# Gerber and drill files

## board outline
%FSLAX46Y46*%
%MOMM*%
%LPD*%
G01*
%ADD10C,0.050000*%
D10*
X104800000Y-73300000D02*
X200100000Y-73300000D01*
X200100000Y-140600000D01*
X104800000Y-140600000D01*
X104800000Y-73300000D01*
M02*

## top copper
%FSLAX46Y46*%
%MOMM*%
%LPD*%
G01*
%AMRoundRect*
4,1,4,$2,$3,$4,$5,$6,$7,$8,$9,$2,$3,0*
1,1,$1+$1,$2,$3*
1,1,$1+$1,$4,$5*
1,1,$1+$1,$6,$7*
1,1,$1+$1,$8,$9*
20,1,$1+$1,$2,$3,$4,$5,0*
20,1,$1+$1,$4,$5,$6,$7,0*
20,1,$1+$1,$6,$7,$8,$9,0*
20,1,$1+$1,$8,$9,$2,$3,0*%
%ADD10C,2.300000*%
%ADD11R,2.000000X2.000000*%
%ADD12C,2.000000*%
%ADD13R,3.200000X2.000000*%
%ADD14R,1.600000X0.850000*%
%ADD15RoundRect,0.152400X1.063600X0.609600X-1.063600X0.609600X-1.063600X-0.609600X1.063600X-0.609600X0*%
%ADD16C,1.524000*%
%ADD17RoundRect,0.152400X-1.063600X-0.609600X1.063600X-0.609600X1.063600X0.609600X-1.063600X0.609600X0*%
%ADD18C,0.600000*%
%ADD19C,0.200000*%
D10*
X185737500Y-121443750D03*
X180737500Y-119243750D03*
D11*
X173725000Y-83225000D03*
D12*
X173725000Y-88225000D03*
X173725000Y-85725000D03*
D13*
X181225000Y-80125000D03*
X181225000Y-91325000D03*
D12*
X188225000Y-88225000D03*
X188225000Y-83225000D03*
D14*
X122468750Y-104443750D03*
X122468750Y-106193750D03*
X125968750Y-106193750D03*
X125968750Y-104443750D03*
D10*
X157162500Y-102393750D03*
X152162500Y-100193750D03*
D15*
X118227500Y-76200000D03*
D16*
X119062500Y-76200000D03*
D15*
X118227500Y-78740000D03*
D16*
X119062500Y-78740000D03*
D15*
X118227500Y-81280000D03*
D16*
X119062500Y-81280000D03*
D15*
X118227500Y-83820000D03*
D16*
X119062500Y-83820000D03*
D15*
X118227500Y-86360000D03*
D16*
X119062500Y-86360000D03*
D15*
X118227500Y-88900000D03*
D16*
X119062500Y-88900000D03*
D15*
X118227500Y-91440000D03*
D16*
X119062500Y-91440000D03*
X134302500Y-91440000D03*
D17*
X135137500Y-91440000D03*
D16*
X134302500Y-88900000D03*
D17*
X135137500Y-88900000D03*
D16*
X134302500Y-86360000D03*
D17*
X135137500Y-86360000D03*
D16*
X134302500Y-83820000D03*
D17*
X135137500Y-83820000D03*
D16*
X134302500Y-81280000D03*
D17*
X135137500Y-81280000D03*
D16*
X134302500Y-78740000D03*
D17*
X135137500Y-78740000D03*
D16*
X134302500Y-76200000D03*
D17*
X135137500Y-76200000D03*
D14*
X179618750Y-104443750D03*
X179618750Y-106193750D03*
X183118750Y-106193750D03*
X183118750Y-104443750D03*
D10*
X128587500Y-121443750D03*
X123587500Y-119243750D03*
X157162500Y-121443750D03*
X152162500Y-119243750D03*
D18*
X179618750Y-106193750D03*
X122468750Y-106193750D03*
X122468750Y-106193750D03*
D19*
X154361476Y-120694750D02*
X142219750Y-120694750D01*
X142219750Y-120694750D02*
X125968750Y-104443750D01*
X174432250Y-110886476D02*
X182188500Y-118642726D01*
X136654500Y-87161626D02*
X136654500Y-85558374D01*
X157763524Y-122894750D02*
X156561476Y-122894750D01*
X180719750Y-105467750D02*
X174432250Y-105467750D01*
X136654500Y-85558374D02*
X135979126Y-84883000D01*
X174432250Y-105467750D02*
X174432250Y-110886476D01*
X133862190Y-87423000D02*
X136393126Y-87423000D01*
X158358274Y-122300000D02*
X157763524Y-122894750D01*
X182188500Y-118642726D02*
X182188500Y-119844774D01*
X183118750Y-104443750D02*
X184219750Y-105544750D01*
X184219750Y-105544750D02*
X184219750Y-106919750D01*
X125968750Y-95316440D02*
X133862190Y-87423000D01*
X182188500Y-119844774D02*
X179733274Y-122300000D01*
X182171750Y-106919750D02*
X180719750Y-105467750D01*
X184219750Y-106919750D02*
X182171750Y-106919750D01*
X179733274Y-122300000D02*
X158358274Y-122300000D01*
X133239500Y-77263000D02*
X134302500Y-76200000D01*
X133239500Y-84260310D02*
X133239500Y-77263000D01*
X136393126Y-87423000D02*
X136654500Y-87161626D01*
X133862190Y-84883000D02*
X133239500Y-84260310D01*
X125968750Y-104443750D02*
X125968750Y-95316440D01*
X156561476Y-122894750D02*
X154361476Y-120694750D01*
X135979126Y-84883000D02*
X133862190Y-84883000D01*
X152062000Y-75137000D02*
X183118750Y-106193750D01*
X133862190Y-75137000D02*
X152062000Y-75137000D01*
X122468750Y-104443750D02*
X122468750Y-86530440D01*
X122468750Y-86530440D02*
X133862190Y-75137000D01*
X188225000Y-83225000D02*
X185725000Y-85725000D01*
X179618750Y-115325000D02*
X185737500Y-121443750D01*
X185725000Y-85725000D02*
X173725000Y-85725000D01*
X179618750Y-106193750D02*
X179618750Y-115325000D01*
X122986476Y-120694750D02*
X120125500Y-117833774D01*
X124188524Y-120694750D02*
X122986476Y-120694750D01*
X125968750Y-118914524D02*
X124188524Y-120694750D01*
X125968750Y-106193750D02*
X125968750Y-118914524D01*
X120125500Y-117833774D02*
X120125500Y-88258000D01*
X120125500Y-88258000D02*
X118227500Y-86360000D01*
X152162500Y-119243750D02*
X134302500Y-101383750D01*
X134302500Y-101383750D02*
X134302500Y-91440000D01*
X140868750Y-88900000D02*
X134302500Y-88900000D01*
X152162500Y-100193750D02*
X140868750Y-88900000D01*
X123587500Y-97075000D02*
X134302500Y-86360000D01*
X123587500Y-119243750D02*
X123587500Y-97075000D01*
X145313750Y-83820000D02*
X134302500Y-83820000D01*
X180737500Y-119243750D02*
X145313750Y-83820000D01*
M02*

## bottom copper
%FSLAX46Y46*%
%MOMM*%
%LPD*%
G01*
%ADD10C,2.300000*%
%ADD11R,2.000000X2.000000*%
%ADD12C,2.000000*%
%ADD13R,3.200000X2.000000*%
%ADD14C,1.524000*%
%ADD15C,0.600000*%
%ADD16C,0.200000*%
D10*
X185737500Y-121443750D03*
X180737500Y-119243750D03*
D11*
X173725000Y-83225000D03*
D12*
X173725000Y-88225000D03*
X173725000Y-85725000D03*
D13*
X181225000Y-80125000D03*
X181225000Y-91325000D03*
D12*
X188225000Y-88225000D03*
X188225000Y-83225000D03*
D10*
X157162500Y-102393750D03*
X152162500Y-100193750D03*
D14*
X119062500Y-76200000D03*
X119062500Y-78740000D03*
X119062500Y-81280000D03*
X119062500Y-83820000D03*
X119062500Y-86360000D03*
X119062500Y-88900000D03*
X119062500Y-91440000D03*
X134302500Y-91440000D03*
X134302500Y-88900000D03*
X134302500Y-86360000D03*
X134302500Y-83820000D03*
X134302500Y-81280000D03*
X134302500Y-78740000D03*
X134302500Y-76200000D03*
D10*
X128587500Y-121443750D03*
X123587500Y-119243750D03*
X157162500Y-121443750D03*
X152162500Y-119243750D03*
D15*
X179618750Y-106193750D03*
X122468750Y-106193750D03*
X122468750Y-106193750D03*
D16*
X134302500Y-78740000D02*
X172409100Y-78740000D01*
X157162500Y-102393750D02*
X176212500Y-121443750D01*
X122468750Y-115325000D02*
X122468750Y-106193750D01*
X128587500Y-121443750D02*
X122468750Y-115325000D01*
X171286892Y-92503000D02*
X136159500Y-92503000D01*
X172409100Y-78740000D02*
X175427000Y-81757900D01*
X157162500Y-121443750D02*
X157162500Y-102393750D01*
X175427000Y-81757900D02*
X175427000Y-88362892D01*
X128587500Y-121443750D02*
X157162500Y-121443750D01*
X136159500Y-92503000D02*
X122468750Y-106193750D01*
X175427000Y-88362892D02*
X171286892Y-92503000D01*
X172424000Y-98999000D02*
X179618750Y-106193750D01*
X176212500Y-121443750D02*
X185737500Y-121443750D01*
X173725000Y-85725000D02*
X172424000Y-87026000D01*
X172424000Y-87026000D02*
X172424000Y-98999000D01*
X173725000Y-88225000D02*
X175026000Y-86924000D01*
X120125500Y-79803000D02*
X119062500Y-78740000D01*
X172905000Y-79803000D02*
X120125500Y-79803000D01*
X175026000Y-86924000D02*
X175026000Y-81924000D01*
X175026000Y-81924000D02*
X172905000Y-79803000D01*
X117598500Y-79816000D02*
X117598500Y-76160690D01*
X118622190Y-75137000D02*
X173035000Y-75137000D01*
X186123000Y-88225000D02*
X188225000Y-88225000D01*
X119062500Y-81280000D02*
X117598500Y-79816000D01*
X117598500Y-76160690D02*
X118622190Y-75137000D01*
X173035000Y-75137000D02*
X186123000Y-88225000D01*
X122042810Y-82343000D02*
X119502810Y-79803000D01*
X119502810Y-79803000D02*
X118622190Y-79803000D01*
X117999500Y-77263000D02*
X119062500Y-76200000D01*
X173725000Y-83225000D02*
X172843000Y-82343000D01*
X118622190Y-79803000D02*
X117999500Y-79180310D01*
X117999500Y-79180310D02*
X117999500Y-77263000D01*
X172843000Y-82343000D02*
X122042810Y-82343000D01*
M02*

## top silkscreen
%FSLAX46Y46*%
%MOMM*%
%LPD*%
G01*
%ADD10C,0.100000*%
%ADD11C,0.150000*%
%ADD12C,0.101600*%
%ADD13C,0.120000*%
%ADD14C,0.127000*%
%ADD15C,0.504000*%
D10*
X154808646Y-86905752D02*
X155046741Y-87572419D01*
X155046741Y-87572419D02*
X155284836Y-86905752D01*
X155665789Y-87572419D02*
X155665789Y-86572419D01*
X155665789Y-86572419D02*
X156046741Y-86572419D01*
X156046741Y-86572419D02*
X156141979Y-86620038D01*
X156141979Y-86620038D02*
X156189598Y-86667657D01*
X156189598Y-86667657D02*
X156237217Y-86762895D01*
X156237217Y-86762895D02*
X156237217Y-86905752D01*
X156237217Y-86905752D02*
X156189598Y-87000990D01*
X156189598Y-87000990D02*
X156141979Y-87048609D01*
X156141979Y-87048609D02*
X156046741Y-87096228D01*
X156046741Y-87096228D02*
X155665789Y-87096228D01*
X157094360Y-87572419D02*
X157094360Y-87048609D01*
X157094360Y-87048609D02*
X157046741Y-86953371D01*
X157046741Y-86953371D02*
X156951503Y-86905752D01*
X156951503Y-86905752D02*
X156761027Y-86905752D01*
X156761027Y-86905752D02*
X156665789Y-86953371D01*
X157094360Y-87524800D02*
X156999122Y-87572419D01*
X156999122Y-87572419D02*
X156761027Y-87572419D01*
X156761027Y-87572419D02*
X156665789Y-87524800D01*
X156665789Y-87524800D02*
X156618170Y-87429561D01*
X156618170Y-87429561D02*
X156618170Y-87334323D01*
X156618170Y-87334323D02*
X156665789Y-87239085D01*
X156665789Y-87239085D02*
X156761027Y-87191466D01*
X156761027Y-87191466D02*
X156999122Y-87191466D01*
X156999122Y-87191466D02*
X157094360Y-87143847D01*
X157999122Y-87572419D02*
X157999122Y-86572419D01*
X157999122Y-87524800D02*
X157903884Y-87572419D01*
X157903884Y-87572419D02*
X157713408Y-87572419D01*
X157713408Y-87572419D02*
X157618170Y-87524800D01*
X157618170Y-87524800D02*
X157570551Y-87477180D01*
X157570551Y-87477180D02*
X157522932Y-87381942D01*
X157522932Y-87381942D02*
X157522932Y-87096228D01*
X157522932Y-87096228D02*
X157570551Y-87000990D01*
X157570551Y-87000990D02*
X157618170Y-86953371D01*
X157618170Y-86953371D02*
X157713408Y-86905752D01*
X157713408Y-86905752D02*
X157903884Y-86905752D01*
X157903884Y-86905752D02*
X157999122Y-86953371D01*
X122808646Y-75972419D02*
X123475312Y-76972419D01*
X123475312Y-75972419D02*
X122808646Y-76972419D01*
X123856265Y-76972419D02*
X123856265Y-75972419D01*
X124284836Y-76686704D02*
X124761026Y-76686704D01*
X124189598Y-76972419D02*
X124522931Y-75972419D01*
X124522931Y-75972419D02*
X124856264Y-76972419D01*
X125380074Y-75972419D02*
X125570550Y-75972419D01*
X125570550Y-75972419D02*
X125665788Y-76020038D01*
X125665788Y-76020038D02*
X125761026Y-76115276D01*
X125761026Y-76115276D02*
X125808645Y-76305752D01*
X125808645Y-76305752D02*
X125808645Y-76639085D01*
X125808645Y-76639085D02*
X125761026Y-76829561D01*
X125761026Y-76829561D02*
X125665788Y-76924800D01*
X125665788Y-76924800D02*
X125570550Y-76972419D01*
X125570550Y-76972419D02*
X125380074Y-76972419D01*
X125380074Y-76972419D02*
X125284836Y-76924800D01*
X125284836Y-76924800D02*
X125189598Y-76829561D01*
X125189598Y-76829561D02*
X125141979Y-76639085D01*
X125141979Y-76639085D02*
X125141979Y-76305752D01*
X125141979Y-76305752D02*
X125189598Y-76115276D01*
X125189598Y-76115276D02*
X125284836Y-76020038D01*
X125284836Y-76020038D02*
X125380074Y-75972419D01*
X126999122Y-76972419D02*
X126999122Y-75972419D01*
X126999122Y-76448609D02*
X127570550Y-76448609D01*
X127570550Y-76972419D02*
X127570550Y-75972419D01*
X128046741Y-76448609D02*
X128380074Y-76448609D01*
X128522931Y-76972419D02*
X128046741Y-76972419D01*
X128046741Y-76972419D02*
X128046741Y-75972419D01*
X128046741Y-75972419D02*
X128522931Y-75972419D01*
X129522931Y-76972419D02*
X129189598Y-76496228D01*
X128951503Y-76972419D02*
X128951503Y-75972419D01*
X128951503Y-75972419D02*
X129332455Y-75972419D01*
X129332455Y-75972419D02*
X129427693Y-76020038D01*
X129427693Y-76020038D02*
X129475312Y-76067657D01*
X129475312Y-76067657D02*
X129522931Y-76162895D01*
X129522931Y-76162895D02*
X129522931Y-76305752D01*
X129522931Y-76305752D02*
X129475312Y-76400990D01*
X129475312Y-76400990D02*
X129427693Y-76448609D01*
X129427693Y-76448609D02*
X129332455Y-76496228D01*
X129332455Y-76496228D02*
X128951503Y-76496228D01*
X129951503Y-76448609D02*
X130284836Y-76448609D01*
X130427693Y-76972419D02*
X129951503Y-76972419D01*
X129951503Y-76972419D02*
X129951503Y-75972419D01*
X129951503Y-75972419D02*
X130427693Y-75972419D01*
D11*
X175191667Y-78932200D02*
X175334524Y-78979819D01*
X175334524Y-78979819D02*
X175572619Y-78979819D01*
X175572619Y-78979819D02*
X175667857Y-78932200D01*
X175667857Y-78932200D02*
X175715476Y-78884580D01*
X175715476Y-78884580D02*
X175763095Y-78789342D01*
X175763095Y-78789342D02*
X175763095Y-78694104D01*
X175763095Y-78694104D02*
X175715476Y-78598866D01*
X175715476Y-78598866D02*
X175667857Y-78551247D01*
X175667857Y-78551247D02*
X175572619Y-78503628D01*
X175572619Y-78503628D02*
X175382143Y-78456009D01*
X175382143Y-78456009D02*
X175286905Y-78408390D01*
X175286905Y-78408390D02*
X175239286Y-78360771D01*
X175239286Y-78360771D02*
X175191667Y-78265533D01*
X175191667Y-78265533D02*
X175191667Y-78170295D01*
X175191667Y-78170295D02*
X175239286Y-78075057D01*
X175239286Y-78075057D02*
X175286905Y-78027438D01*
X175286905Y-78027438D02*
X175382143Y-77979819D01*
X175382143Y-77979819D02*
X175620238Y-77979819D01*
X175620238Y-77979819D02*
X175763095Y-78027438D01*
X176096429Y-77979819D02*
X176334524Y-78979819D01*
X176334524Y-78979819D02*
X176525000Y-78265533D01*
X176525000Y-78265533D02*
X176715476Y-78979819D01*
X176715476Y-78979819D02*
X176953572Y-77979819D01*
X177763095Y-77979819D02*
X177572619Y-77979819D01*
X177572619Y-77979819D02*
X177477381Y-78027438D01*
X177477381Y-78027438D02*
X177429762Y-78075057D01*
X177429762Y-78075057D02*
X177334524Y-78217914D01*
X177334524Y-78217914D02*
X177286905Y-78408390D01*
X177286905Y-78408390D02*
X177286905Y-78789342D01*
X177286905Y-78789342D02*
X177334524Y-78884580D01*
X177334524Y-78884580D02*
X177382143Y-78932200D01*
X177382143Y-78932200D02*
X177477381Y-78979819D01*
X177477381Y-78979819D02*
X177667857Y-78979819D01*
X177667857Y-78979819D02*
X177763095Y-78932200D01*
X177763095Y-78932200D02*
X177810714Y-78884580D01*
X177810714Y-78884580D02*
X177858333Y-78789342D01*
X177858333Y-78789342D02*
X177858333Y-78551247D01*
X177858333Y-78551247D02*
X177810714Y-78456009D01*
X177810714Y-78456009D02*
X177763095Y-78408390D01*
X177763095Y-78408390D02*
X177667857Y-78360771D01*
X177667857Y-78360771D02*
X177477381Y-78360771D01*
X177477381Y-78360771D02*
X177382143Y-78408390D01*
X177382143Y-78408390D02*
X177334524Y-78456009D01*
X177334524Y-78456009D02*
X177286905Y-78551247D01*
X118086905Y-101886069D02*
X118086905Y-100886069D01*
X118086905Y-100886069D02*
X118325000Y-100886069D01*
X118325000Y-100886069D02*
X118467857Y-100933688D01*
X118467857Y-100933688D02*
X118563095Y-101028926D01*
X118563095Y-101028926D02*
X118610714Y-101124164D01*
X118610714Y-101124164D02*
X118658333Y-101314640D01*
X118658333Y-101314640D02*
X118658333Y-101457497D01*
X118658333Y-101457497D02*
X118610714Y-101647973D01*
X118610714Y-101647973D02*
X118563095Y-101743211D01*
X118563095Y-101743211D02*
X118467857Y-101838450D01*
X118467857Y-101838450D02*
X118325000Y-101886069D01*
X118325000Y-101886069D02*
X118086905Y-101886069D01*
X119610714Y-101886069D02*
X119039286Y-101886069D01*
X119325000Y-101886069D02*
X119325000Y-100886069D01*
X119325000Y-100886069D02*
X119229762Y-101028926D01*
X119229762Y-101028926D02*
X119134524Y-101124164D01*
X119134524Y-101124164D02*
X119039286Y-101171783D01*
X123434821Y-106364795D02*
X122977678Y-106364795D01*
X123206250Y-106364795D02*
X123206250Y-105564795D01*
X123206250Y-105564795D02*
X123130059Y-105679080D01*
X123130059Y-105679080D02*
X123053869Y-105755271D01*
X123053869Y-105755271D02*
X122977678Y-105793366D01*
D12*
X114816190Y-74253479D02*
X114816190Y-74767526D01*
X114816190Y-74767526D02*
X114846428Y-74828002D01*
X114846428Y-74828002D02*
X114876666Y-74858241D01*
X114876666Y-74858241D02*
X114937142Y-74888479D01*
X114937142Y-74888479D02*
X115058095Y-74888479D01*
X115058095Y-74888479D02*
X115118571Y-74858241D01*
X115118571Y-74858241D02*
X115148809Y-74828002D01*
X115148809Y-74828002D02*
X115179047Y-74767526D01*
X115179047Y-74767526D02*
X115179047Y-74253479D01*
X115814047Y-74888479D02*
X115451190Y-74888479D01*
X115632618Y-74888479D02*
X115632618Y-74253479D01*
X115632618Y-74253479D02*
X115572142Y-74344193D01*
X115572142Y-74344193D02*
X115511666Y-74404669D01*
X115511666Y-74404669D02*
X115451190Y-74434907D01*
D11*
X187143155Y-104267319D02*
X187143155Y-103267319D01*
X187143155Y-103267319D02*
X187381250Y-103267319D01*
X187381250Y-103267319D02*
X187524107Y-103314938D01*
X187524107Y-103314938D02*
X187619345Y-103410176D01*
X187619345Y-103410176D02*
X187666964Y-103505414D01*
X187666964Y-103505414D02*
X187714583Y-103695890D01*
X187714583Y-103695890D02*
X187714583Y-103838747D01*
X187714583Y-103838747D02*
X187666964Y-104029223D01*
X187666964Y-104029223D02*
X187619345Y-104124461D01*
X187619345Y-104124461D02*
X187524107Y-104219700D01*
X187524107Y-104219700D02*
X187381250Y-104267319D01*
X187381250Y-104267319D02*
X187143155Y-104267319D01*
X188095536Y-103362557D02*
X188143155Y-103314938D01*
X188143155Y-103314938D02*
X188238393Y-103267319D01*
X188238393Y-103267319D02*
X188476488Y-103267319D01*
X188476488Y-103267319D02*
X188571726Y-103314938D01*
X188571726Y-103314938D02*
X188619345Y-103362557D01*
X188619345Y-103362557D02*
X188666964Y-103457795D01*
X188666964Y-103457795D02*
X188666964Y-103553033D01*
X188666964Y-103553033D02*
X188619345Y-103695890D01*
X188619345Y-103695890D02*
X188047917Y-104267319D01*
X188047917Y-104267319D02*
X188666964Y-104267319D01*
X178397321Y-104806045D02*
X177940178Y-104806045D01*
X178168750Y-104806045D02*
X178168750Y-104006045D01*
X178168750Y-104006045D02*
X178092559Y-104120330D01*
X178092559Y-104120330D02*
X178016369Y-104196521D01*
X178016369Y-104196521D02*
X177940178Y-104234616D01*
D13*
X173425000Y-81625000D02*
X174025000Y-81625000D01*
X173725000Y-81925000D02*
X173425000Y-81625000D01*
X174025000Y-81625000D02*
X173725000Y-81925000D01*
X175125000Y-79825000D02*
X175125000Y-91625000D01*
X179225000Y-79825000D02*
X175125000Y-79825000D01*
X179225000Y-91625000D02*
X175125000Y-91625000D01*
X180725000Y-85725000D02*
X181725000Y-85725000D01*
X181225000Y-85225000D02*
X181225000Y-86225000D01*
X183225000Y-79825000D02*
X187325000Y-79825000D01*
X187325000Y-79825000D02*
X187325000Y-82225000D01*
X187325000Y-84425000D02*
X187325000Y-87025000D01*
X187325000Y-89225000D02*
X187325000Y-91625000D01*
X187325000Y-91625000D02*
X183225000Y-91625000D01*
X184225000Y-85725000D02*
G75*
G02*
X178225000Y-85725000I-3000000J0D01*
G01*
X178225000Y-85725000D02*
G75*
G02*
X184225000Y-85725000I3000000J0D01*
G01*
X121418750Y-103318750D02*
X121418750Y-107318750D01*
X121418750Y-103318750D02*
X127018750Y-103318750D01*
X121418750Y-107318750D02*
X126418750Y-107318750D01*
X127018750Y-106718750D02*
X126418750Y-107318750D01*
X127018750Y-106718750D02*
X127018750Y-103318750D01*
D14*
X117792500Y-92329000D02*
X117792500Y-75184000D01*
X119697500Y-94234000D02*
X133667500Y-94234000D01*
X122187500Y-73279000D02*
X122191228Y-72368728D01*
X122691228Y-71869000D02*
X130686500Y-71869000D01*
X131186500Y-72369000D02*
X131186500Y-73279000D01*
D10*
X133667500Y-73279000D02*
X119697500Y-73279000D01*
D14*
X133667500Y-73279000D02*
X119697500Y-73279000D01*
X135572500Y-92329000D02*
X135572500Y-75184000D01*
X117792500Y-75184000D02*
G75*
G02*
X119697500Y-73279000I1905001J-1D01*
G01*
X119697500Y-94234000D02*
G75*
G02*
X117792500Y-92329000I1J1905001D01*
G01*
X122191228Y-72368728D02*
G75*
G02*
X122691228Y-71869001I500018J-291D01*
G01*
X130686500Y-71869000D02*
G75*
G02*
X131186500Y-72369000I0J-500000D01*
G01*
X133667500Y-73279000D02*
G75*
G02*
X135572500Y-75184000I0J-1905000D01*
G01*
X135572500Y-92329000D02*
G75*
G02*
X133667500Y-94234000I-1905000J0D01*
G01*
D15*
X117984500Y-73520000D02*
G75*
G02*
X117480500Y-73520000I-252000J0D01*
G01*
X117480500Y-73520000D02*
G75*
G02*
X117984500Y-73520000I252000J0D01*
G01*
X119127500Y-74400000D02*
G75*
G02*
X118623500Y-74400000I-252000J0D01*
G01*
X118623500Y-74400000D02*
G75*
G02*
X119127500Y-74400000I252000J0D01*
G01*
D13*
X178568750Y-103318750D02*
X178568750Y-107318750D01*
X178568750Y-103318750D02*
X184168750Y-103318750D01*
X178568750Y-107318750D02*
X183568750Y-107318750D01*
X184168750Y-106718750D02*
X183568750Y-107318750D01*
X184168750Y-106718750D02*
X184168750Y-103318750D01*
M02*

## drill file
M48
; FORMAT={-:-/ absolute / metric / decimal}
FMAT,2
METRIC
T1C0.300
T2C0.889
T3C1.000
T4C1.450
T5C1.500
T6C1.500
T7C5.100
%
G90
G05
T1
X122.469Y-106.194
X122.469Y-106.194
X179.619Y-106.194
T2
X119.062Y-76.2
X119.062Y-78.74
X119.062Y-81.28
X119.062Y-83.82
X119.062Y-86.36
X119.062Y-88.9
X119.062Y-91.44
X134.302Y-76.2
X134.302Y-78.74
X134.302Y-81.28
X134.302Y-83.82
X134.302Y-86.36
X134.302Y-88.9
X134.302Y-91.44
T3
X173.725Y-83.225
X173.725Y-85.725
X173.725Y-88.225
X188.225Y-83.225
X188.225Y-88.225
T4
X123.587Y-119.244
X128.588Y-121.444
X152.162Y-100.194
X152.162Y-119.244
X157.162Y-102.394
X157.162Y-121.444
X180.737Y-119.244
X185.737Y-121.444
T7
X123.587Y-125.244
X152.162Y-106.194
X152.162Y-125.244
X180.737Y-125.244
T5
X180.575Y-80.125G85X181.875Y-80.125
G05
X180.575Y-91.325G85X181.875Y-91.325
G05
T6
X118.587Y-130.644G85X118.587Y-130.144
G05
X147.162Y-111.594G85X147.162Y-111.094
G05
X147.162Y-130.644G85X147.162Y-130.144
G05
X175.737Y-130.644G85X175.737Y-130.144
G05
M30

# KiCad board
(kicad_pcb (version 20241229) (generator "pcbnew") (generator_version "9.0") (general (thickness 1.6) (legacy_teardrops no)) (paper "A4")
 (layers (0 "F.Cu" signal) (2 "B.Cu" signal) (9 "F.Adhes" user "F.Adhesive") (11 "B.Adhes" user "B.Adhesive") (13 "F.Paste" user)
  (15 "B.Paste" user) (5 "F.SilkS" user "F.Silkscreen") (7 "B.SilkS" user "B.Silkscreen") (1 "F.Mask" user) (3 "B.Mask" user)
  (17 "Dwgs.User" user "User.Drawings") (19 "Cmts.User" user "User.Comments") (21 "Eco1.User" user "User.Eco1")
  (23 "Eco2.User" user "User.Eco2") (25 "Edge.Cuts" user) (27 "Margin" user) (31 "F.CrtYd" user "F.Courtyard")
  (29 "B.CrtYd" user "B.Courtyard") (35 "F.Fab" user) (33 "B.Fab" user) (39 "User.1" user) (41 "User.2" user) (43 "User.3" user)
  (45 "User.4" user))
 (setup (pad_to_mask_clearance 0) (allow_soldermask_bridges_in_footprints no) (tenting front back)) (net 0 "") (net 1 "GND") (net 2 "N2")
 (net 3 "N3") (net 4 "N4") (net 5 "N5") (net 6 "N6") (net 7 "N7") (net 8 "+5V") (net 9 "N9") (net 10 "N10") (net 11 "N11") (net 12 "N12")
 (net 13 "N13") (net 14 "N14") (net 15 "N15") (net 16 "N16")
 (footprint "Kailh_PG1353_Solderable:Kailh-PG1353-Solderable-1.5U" (layer "F.Cu") (at 180.7375 125.24375)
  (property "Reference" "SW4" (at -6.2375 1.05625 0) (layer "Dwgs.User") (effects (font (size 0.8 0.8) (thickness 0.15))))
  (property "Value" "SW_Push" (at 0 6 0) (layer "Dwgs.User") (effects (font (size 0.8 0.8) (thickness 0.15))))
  (pad "" np_thru_hole oval (at -5 5.15 180) (size 1.5 2) (drill oval 1.5 2) (layers "*.Cu" "*.Mask"))
  (pad "" np_thru_hole circle (at 0 0 180) (size 5 5) (drill 5.1) (layers "*.Cu" "*.Mask"))
  (pad "1" thru_hole circle (at 5 -3.8 180) (size 2.3 2.3) (drill 1.45) (layers "*.Cu" "B.Mask") (remove_unused_layers no) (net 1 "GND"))
  (pad "2" thru_hole circle (at 0 -6 180) (size 2.3 2.3) (drill 1.45) (layers "*.Cu" "B.Mask") (remove_unused_layers no) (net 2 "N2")))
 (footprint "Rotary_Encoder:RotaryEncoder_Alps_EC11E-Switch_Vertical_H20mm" (layer "F.Cu") (at 173.725 83.225)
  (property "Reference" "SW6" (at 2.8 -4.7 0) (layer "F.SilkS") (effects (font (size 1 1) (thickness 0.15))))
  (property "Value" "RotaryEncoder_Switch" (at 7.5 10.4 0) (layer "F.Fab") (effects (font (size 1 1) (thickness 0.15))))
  (fp_line (start -0.3 -1.6) (end 0.3 -1.6) (stroke (width 0.12) (type solid)) (layer "F.SilkS"))
  (fp_line (start 0 -1.3) (end -0.3 -1.6) (stroke (width 0.12) (type solid)) (layer "F.SilkS"))
  (fp_line (start 0.3 -1.6) (end 0 -1.3) (stroke (width 0.12) (type solid)) (layer "F.SilkS"))
  (fp_line (start 1.4 -3.4) (end 1.4 8.4) (stroke (width 0.12) (type solid)) (layer "F.SilkS"))
  (fp_line (start 5.5 -3.4) (end 1.4 -3.4) (stroke (width 0.12) (type solid)) (layer "F.SilkS"))
  (fp_line (start 5.5 8.4) (end 1.4 8.4) (stroke (width 0.12) (type solid)) (layer "F.SilkS"))
  (fp_line (start 7 2.5) (end 8 2.5) (stroke (width 0.12) (type solid)) (layer "F.SilkS"))
  (fp_line (start 7.5 2) (end 7.5 3) (stroke (width 0.12) (type solid)) (layer "F.SilkS"))
  (fp_line (start 9.5 -3.4) (end 13.6 -3.4) (stroke (width 0.12) (type solid)) (layer "F.SilkS"))
  (fp_line (start 13.6 -3.4) (end 13.6 -1) (stroke (width 0.12) (type solid)) (layer "F.SilkS"))
  (fp_line (start 13.6 1.2) (end 13.6 3.8) (stroke (width 0.12) (type solid)) (layer "F.SilkS"))
  (fp_line (start 13.6 6) (end 13.6 8.4) (stroke (width 0.12) (type solid)) (layer "F.SilkS"))
  (fp_line (start 13.6 8.4) (end 9.5 8.4) (stroke (width 0.12) (type solid)) (layer "F.SilkS"))
  (fp_circle (center 7.5 2.5) (end 10.5 2.5) (stroke (width 0.12) (type solid)) (fill no) (layer "F.SilkS"))
  (pad "A" thru_hole rect (at 0 0) (size 2 2) (drill 1) (layers "*.Cu" "*.Mask") (remove_unused_layers no) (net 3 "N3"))
  (pad "B" thru_hole circle (at 0 5) (size 2 2) (drill 1) (layers "*.Cu" "*.Mask") (remove_unused_layers no) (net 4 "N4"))
  (pad "C" thru_hole circle (at 0 2.5) (size 2 2) (drill 1) (layers "*.Cu" "*.Mask") (remove_unused_layers no) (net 1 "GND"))
  (pad "MP" thru_hole rect (at 7.5 -3.1) (size 3.2 2) (drill oval 2.8 1.5) (layers "*.Cu" "*.Mask") (remove_unused_layers no))
  (pad "MP" thru_hole rect (at 7.5 8.1) (size 3.2 2) (drill oval 2.8 1.5) (layers "*.Cu" "*.Mask") (remove_unused_layers no))
  (pad "S1" thru_hole circle (at 14.5 5) (size 2 2) (drill 1) (layers "*.Cu" "*.Mask") (remove_unused_layers no) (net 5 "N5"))
  (pad "S2" thru_hole circle (at 14.5 0) (size 2 2) (drill 1) (layers "*.Cu" "*.Mask") (remove_unused_layers no) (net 1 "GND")))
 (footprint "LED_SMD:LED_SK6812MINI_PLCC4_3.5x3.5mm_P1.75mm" (layer "F.Cu") (at 124.21875 105.31875)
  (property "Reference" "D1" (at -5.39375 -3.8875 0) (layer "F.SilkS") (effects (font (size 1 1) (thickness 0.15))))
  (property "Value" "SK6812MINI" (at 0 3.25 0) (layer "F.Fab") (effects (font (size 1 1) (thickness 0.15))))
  (fp_line (start -2.8 -2) (end -2.8 2) (stroke (width 0.12) (type default)) (layer "F.SilkS"))
  (fp_line (start -2.8 -2) (end 2.8 -2) (stroke (width 0.12) (type solid)) (layer "F.SilkS"))
  (fp_line (start -2.8 2) (end 2.2 2) (stroke (width 0.12) (type solid)) (layer "F.SilkS"))
  (fp_line (start 2.8 1.4) (end 2.2 2) (stroke (width 0.12) (type default)) (layer "F.SilkS"))
  (fp_line (start 2.8 1.4) (end 2.8 -2) (stroke (width 0.12) (type solid)) (layer "F.SilkS"))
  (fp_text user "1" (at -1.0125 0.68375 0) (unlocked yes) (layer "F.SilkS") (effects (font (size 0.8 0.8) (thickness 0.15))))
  (pad "1" smd rect (at -1.75 -0.875) (size 1.6 0.85) (layers "F.Cu" "F.Mask" "F.Paste") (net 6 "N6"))
  (pad "2" smd rect (at -1.75 0.875) (size 1.6 0.85) (layers "F.Cu" "F.Mask" "F.Paste") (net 1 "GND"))
  (pad "3" smd rect (at 1.75 0.875) (size 1.6 0.85) (layers "F.Cu" "F.Mask" "F.Paste") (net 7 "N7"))
  (pad "4" smd rect (at 1.75 -0.875) (size 1.6 0.85) (layers "F.Cu" "F.Mask" "F.Paste") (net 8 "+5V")))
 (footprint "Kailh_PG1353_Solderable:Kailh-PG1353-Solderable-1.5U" (layer "F.Cu") (at 152.1625 106.19375)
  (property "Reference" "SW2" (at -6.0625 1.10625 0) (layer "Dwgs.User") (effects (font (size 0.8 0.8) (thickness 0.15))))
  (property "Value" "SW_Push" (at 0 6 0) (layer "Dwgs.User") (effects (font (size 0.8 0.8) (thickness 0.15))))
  (pad "" np_thru_hole oval (at -5 5.15 180) (size 1.5 2) (drill oval 1.5 2) (layers "*.Cu" "*.Mask"))
  (pad "" np_thru_hole circle (at 0 0 180) (size 5 5) (drill 5.1) (layers "*.Cu" "*.Mask"))
  (pad "1" thru_hole circle (at 5 -3.8 180) (size 2.3 2.3) (drill 1.45) (layers "*.Cu" "B.Mask") (remove_unused_layers no) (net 1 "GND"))
  (pad "2" thru_hole circle (at 0 -6 180) (size 2.3 2.3) (drill 1.45) (layers "*.Cu" "B.Mask") (remove_unused_layers no) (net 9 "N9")))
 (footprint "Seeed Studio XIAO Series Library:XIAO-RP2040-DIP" (layer "F.Cu") (at 126.6825 83.82)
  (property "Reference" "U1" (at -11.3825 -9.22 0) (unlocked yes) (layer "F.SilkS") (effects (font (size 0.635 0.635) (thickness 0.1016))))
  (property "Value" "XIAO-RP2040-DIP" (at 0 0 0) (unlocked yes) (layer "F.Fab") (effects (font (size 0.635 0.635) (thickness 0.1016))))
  (fp_line (start -8.89 8.509) (end -8.89 -8.636) (stroke (width 0.127) (type solid)) (layer "F.SilkS"))
  (fp_line (start -6.985 10.414) (end 6.985 10.414) (stroke (width 0.127) (type solid)) (layer "F.SilkS"))
  (fp_line (start -4.495 -10.541) (end -4.491272 -11.451272) (stroke (width 0.127) (type solid)) (layer "F.SilkS"))
  (fp_line (start -3.991272 -11.951) (end 4.004 -11.951) (stroke (width 0.127) (type solid)) (layer "F.SilkS"))
  (fp_line (start 4.504 -11.451) (end 4.504 -10.541) (stroke (width 0.127) (type solid)) (layer "F.SilkS"))
  (fp_line (start 6.985 -10.541) (end -6.985 -10.541) (stroke (width 0.1) (type solid)) (layer "F.SilkS"))
  (fp_line (start 6.985 -10.541) (end -6.985 -10.541) (stroke (width 0.127) (type solid)) (layer "F.SilkS"))
  (fp_line (start 8.89 8.509) (end 8.89 -8.636) (stroke (width 0.127) (type solid)) (layer "F.SilkS"))
  (fp_arc (start -8.89 -8.636) (mid -8.332038 -9.983038) (end -6.985 -10.541) (stroke (width 0.127) (type solid)) (layer "F.SilkS"))
  (fp_arc (start -6.985 10.414) (mid -8.332038 9.856038) (end -8.89 8.509) (stroke (width 0.127) (type solid)) (layer "F.SilkS"))
  (fp_arc (start -4.491272 -11.451272) (mid -4.344728 -11.80464) (end -3.991272 -11.951) (stroke (width 0.127) (type default))
   (layer "F.SilkS"))
  (fp_arc (start 4.004 -11.951) (mid 4.357553 -11.804553) (end 4.504 -11.451) (stroke (width 0.127) (type default)) (layer "F.SilkS"))
  (fp_arc (start 6.985 -10.541) (mid 8.332038 -9.983038) (end 8.89 -8.636) (stroke (width 0.127) (type solid)) (layer "F.SilkS"))
  (fp_arc (start 8.89 8.509) (mid 8.332038 9.856038) (end 6.985 10.414) (stroke (width 0.127) (type solid)) (layer "F.SilkS"))
  (fp_circle (center -8.95 -10.3) (end -8.95 -10.554) (stroke (width 0.5) (type solid)) (fill yes) (layer "F.SilkS"))
  (fp_circle (center -7.807 -9.42) (end -7.807 -9.674) (stroke (width 0.5) (type solid)) (fill yes) (layer "F.SilkS"))
  (pad "1" smd roundrect (at -8.455 -7.62 180) (size 2.432 1.524) (layers "F.Cu" "F.Mask") (roundrect_rratio 0.1) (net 3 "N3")
   (thermal_bridge_angle 45))
  (pad "1" thru_hole circle (at -7.62 -7.62 180) (size 1.524 1.524) (drill 0.889) (layers "*.Cu" "*.Mask") (remove_unused_layers no)
   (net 3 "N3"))
  (pad "2" smd roundrect (at -8.455 -5.08 180) (size 2.432 1.524) (layers "F.Cu" "F.Mask") (roundrect_rratio 0.1) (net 4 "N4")
   (thermal_bridge_angle 45))
  (pad "2" thru_hole circle (at -7.62 -5.08 180) (size 1.524 1.524) (drill 0.889) (layers "*.Cu" "*.Mask") (remove_unused_layers no)
   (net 4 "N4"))
  (pad "3" smd roundrect (at -8.455 -2.54 180) (size 2.432 1.524) (layers "F.Cu" "F.Mask") (roundrect_rratio 0.1) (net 5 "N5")
   (thermal_bridge_angle 45))
  (pad "3" thru_hole circle (at -7.62 -2.54 180) (size 1.524 1.524) (drill 0.889) (layers "*.Cu" "*.Mask") (remove_unused_layers no)
   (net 5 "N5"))
  (pad "4" smd roundrect (at -8.455 0 180) (size 2.432 1.524) (layers "F.Cu" "F.Mask") (roundrect_rratio 0.1) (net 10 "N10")
   (thermal_bridge_angle 45))
  (pad "4" thru_hole circle (at -7.62 0 180) (size 1.524 1.524) (drill 0.889) (layers "*.Cu" "*.Mask") (remove_unused_layers no)
   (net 10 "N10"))
  (pad "5" smd roundrect (at -8.455 2.54 180) (size 2.432 1.524) (layers "F.Cu" "F.Mask") (roundrect_rratio 0.1) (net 7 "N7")
   (thermal_bridge_angle 45))
  (pad "5" thru_hole circle (at -7.62 2.54 180) (size 1.524 1.524) (drill 0.889) (layers "*.Cu" "*.Mask") (remove_unused_layers no)
   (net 7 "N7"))
  (pad "6" smd roundrect (at -8.455 5.08 180) (size 2.432 1.524) (layers "F.Cu" "F.Mask") (roundrect_rratio 0.1) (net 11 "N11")
   (thermal_bridge_angle 45))
  (pad "6" thru_hole circle (at -7.62 5.08 180) (size 1.524 1.524) (drill 0.889) (layers "*.Cu" "*.Mask") (remove_unused_layers no)
   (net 11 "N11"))
  (pad "7" smd roundrect (at -8.455 7.62 180) (size 2.432 1.524) (layers "F.Cu" "F.Mask") (roundrect_rratio 0.1) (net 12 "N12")
   (thermal_bridge_angle 45))
  (pad "7" thru_hole circle (at -7.62 7.62 180) (size 1.524 1.524) (drill 0.889) (layers "*.Cu" "*.Mask") (remove_unused_layers no)
   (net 12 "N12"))
  (pad "8" thru_hole circle (at 7.62 7.62) (size 1.524 1.524) (drill 0.889) (layers "*.Cu" "*.Mask") (remove_unused_layers no)
   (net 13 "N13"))
  (pad "8" smd roundrect (at 8.455 7.62) (size 2.432 1.524) (layers "F.Cu" "F.Mask") (roundrect_rratio 0.1) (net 13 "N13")
   (thermal_bridge_angle 45))
  (pad "9" thru_hole circle (at 7.62 5.08) (size 1.524 1.524) (drill 0.889) (layers "*.Cu" "*.Mask") (remove_unused_layers no) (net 9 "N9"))
  (pad "9" smd roundrect (at 8.455 5.08) (size 2.432 1.524) (layers "F.Cu" "F.Mask") (roundrect_rratio 0.1) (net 9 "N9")
   (thermal_bridge_angle 45))
  (pad "10" thru_hole circle (at 7.62 2.54) (size 1.524 1.524) (drill 0.889) (layers "*.Cu" "*.Mask") (remove_unused_layers no)
   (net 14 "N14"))
  (pad "10" smd roundrect (at 8.455 2.54) (size 2.432 1.524) (layers "F.Cu" "F.Mask") (roundrect_rratio 0.1) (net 14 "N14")
   (thermal_bridge_angle 45))
  (pad "11" thru_hole circle (at 7.62 0) (size 1.524 1.524) (drill 0.889) (layers "*.Cu" "*.Mask") (remove_unused_layers no) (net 2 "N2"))
  (pad "11" smd roundrect (at 8.455 0) (size 2.432 1.524) (layers "F.Cu" "F.Mask") (roundrect_rratio 0.1) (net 2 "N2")
   (thermal_bridge_angle 45))
  (pad "12" thru_hole circle (at 7.62 -2.54) (size 1.524 1.524) (drill 0.889) (layers "*.Cu" "*.Mask") (remove_unused_layers no)
   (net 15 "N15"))
  (pad "12" smd roundrect (at 8.455 -2.54) (size 2.432 1.524) (layers "F.Cu" "F.Mask") (roundrect_rratio 0.1) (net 15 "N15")
   (thermal_bridge_angle 45))
  (pad "13" thru_hole circle (at 7.62 -5.08) (size 1.524 1.524) (drill 0.889) (layers "*.Cu" "*.Mask") (remove_unused_layers no)
   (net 1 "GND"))
  (pad "13" smd roundrect (at 8.455 -5.08) (size 2.432 1.524) (layers "F.Cu" "F.Mask") (roundrect_rratio 0.1) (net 1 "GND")
   (thermal_bridge_angle 45))
  (pad "14" thru_hole circle (at 7.62 -7.62) (size 1.524 1.524) (drill 0.889) (layers "*.Cu" "*.Mask") (remove_unused_layers no)
   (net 8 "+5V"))
  (pad "14" smd roundrect (at 8.455 -7.62) (size 2.432 1.524) (layers "F.Cu" "F.Mask") (roundrect_rratio 0.1) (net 8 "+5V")
   (thermal_bridge_angle 45)))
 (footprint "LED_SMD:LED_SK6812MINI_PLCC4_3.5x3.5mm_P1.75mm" (layer "F.Cu") (at 181.36875 105.31875)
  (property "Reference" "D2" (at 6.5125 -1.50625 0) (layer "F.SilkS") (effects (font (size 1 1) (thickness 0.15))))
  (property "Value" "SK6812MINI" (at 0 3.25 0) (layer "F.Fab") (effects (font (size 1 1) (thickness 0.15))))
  (fp_line (start -2.8 -2) (end -2.8 2) (stroke (width 0.12) (type default)) (layer "F.SilkS"))
  (fp_line (start -2.8 -2) (end 2.8 -2) (stroke (width 0.12) (type solid)) (layer "F.SilkS"))
  (fp_line (start -2.8 2) (end 2.2 2) (stroke (width 0.12) (type solid)) (layer "F.SilkS"))
  (fp_line (start 2.8 1.4) (end 2.2 2) (stroke (width 0.12) (type default)) (layer "F.SilkS"))
  (fp_line (start 2.8 1.4) (end 2.8 -2) (stroke (width 0.12) (type solid)) (layer "F.SilkS"))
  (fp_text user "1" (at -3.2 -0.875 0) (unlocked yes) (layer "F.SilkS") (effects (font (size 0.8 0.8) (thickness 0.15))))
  (pad "1" smd rect (at -1.75 -0.875) (size 1.6 0.85) (layers "F.Cu" "F.Mask" "F.Paste") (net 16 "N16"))
  (pad "2" smd rect (at -1.75 0.875) (size 1.6 0.85) (layers "F.Cu" "F.Mask" "F.Paste") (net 1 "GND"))
  (pad "3" smd rect (at 1.75 0.875) (size 1.6 0.85) (layers "F.Cu" "F.Mask" "F.Paste") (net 6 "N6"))
  (pad "4" smd rect (at 1.75 -0.875) (size 1.6 0.85) (layers "F.Cu" "F.Mask" "F.Paste") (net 8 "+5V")))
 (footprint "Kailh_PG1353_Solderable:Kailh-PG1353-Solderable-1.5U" (layer "F.Cu") (at 123.5875 125.24375)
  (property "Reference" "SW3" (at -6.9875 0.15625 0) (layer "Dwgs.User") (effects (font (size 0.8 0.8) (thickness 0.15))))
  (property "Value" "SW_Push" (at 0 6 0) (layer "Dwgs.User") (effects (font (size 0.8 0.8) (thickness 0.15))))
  (pad "" np_thru_hole oval (at -5 5.15 180) (size 1.5 2) (drill oval 1.5 2) (layers "*.Cu" "*.Mask"))
  (pad "" np_thru_hole circle (at 0 0 180) (size 5 5) (drill 5.1) (layers "*.Cu" "*.Mask"))
  (pad "1" thru_hole circle (at 5 -3.8 180) (size 2.3 2.3) (drill 1.45) (layers "*.Cu" "B.Mask") (remove_unused_layers no) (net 1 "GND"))
  (pad "2" thru_hole circle (at 0 -6 180) (size 2.3 2.3) (drill 1.45) (layers "*.Cu" "B.Mask") (remove_unused_layers no) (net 14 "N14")))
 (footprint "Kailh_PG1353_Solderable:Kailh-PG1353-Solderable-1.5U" (layer "F.Cu") (at 152.1625 125.24375)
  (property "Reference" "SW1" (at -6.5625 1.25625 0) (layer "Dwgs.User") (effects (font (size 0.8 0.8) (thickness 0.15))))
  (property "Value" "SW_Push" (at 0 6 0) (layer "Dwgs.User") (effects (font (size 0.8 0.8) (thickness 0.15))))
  (pad "" np_thru_hole oval (at -5 5.15 180) (size 1.5 2) (drill oval 1.5 2) (layers "*.Cu" "*.Mask"))
  (pad "" np_thru_hole circle (at 0 0 180) (size 5 5) (drill 5.1) (layers "*.Cu" "*.Mask"))
  (pad "1" thru_hole circle (at 5 -3.8 180) (size 2.3 2.3) (drill 1.45) (layers "*.Cu" "B.Mask") (remove_unused_layers no) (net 1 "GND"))
  (pad "2" thru_hole circle (at 0 -6 180) (size 2.3 2.3) (drill 1.45) (layers "*.Cu" "B.Mask") (remove_unused_layers no) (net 13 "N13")))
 (gr_rect (start 104.8 73.3) (end 200.1 140.6) (stroke (width 0.05) (type default)) (fill no) (layer "Edge.Cuts"))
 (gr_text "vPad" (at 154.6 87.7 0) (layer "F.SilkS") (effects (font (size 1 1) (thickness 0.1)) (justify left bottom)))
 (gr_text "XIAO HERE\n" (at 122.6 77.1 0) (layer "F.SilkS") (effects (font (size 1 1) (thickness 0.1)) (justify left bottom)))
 (segment (start 154.361476 120.69475) (end 142.21975 120.69475) (width 0.2) (layer "F.Cu") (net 8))
 (segment (start 142.21975 120.69475) (end 125.96875 104.44375) (width 0.2) (layer "F.Cu") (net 8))
 (segment (start 174.43225 110.886476) (end 182.1885 118.642726) (width 0.2) (layer "F.Cu") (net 8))
 (segment (start 136.6545 87.161626) (end 136.6545 85.558374) (width 0.2) (layer "F.Cu") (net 8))
 (segment (start 157.763524 122.89475) (end 156.561476 122.89475) (width 0.2) (layer "F.Cu") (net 8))
 (segment (start 180.71975 105.46775) (end 174.43225 105.46775) (width 0.2) (layer "F.Cu") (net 8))
 (segment (start 136.6545 85.558374) (end 135.979126 84.883) (width 0.2) (layer "F.Cu") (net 8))
 (segment (start 174.43225 105.46775) (end 174.43225 110.886476) (width 0.2) (layer "F.Cu") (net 8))
 (segment (start 133.86219 87.423) (end 136.393126 87.423) (width 0.2) (layer "F.Cu") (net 8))
 (segment (start 158.358274 122.3) (end 157.763524 122.89475) (width 0.2) (layer "F.Cu") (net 8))
 (segment (start 182.1885 118.642726) (end 182.1885 119.844774) (width 0.2) (layer "F.Cu") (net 8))
 (segment (start 183.11875 104.44375) (end 184.21975 105.54475) (width 0.2) (layer "F.Cu") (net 8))
 (segment (start 184.21975 105.54475) (end 184.21975 106.91975) (width 0.2) (layer "F.Cu") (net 8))
 (segment (start 125.96875 95.31644) (end 133.86219 87.423) (width 0.2) (layer "F.Cu") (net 8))
 (segment (start 182.1885 119.844774) (end 179.733274 122.3) (width 0.2) (layer "F.Cu") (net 8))
 (segment (start 182.17175 106.91975) (end 180.71975 105.46775) (width 0.2) (layer "F.Cu") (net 8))
 (segment (start 184.21975 106.91975) (end 182.17175 106.91975) (width 0.2) (layer "F.Cu") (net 8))
 (segment (start 179.733274 122.3) (end 158.358274 122.3) (width 0.2) (layer "F.Cu") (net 8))
 (segment (start 133.2395 77.263) (end 134.3025 76.2) (width 0.2) (layer "F.Cu") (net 8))
 (segment (start 133.2395 84.26031) (end 133.2395 77.263) (width 0.2) (layer "F.Cu") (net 8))
 (segment (start 136.393126 87.423) (end 136.6545 87.161626) (width 0.2) (layer "F.Cu") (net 8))
 (segment (start 133.86219 84.883) (end 133.2395 84.26031) (width 0.2) (layer "F.Cu") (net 8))
 (segment (start 125.96875 104.44375) (end 125.96875 95.31644) (width 0.2) (layer "F.Cu") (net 8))
 (segment (start 156.561476 122.89475) (end 154.361476 120.69475) (width 0.2) (layer "F.Cu") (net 8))
 (segment (start 135.979126 84.883) (end 133.86219 84.883) (width 0.2) (layer "F.Cu") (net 8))
 (segment (start 152.062 75.137) (end 183.11875 106.19375) (width 0.2) (layer "F.Cu") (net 6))
 (segment (start 133.86219 75.137) (end 152.062 75.137) (width 0.2) (layer "F.Cu") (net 6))
 (segment (start 122.46875 104.44375) (end 122.46875 86.53044) (width 0.2) (layer "F.Cu") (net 6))
 (segment (start 122.46875 86.53044) (end 133.86219 75.137) (width 0.2) (layer "F.Cu") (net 6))
 (segment (start 188.225 83.225) (end 185.725 85.725) (width 0.2) (layer "F.Cu") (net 1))
 (segment (start 179.61875 115.325) (end 185.7375 121.44375) (width 0.2) (layer "F.Cu") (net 1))
 (segment (start 185.725 85.725) (end 173.725 85.725) (width 0.2) (layer "F.Cu") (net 1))
 (segment (start 179.61875 106.19375) (end 179.61875 115.325) (width 0.2) (layer "F.Cu") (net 1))
 (via (at 179.61875 106.19375) (size 0.6) (drill 0.3) (layers "F.Cu" "B.Cu") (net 1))
 (via (at 122.46875 106.19375) (size 0.6) (drill 0.3) (layers "F.Cu" "B.Cu") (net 1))
 (via (at 122.46875 106.19375) (size 0.6) (drill 0.3) (layers "F.Cu" "B.Cu") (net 1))
 (segment (start 134.3025 78.74) (end 172.4091 78.74) (width 0.2) (layer "B.Cu") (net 1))
 (segment (start 157.1625 102.39375) (end 176.2125 121.44375) (width 0.2) (layer "B.Cu") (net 1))
 (segment (start 122.46875 115.325) (end 122.46875 106.19375) (width 0.2) (layer "B.Cu") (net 1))
 (segment (start 128.5875 121.44375) (end 122.46875 115.325) (width 0.2) (layer "B.Cu") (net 1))
 (segment (start 171.286892 92.503) (end 136.1595 92.503) (width 0.2) (layer "B.Cu") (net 1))
 (segment (start 172.4091 78.74) (end 175.427 81.7579) (width 0.2) (layer "B.Cu") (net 1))
 (segment (start 157.1625 121.44375) (end 157.1625 102.39375) (width 0.2) (layer "B.Cu") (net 1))
 (segment (start 175.427 81.7579) (end 175.427 88.362892) (width 0.2) (layer "B.Cu") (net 1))
 (segment (start 128.5875 121.44375) (end 157.1625 121.44375) (width 0.2) (layer "B.Cu") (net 1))
 (segment (start 136.1595 92.503) (end 122.46875 106.19375) (width 0.2) (layer "B.Cu") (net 1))
 (segment (start 175.427 88.362892) (end 171.286892 92.503) (width 0.2) (layer "B.Cu") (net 1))
 (segment (start 172.424 98.999) (end 179.61875 106.19375) (width 0.2) (layer "B.Cu") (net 1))
 (segment (start 176.2125 121.44375) (end 185.7375 121.44375) (width 0.2) (layer "B.Cu") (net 1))
 (segment (start 173.725 85.725) (end 172.424 87.026) (width 0.2) (layer "B.Cu") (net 1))
 (segment (start 172.424 87.026) (end 172.424 98.999) (width 0.2) (layer "B.Cu") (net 1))
 (segment (start 122.986476 120.69475) (end 120.1255 117.833774) (width 0.2) (layer "F.Cu") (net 7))
 (segment (start 124.188524 120.69475) (end 122.986476 120.69475) (width 0.2) (layer "F.Cu") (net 7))
 (segment (start 125.96875 118.914524) (end 124.188524 120.69475) (width 0.2) (layer "F.Cu") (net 7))
 (segment (start 125.96875 106.19375) (end 125.96875 118.914524) (width 0.2) (layer "F.Cu") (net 7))
 (segment (start 120.1255 117.833774) (end 120.1255 88.258) (width 0.2) (layer "F.Cu") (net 7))
 (segment (start 120.1255 88.258) (end 118.2275 86.36) (width 0.2) (layer "F.Cu") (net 7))
 (segment (start 152.1625 119.24375) (end 134.3025 101.38375) (width 0.2) (layer "F.Cu") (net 13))
 (segment (start 134.3025 101.38375) (end 134.3025 91.44) (width 0.2) (layer "F.Cu") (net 13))
 (segment (start 140.86875 88.9) (end 134.3025 88.9) (width 0.2) (layer "F.Cu") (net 9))
 (segment (start 152.1625 100.19375) (end 140.86875 88.9) (width 0.2) (layer "F.Cu") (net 9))
 (segment (start 123.5875 97.075) (end 134.3025 86.36) (width 0.2) (layer "F.Cu") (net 14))
 (segment (start 123.5875 119.24375) (end 123.5875 97.075) (width 0.2) (layer "F.Cu") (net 14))
 (segment (start 145.31375 83.82) (end 134.3025 83.82) (width 0.2) (layer "F.Cu") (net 2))
 (segment (start 180.7375 119.24375) (end 145.31375 83.82) (width 0.2) (layer "F.Cu") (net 2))
 (segment (start 173.725 88.225) (end 175.026 86.924) (width 0.2) (layer "B.Cu") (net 4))
 (segment (start 120.1255 79.803) (end 119.0625 78.74) (width 0.2) (layer "B.Cu") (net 4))
 (segment (start 172.905 79.803) (end 120.1255 79.803) (width 0.2) (layer "B.Cu") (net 4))
 (segment (start 175.026 86.924) (end 175.026 81.924) (width 0.2) (layer "B.Cu") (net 4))
 (segment (start 175.026 81.924) (end 172.905 79.803) (width 0.2) (layer "B.Cu") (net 4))
 (segment (start 117.5985 79.816) (end 117.5985 76.16069) (width 0.2) (layer "B.Cu") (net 5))
 (segment (start 118.62219 75.137) (end 173.035 75.137) (width 0.2) (layer "B.Cu") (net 5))
 (segment (start 186.123 88.225) (end 188.225 88.225) (width 0.2) (layer "B.Cu") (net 5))
 (segment (start 119.0625 81.28) (end 117.5985 79.816) (width 0.2) (layer "B.Cu") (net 5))
 (segment (start 117.5985 76.16069) (end 118.62219 75.137) (width 0.2) (layer "B.Cu") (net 5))
 (segment (start 173.035 75.137) (end 186.123 88.225) (width 0.2) (layer "B.Cu") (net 5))
 (segment (start 122.04281 82.343) (end 119.50281 79.803) (width 0.2) (layer "B.Cu") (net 3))
 (segment (start 119.50281 79.803) (end 118.62219 79.803) (width 0.2) (layer "B.Cu") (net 3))
 (segment (start 117.9995 77.263) (end 119.0625 76.2) (width 0.2) (layer "B.Cu") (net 3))
 (segment (start 173.725 83.225) (end 172.843 82.343) (width 0.2) (layer "B.Cu") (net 3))
 (segment (start 118.62219 79.803) (end 117.9995 79.18031) (width 0.2) (layer "B.Cu") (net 3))
 (segment (start 117.9995 79.18031) (end 117.9995 77.263) (width 0.2) (layer "B.Cu") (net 3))
 (segment (start 172.843 82.343) (end 122.04281 82.343) (width 0.2) (layer "B.Cu") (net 3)))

